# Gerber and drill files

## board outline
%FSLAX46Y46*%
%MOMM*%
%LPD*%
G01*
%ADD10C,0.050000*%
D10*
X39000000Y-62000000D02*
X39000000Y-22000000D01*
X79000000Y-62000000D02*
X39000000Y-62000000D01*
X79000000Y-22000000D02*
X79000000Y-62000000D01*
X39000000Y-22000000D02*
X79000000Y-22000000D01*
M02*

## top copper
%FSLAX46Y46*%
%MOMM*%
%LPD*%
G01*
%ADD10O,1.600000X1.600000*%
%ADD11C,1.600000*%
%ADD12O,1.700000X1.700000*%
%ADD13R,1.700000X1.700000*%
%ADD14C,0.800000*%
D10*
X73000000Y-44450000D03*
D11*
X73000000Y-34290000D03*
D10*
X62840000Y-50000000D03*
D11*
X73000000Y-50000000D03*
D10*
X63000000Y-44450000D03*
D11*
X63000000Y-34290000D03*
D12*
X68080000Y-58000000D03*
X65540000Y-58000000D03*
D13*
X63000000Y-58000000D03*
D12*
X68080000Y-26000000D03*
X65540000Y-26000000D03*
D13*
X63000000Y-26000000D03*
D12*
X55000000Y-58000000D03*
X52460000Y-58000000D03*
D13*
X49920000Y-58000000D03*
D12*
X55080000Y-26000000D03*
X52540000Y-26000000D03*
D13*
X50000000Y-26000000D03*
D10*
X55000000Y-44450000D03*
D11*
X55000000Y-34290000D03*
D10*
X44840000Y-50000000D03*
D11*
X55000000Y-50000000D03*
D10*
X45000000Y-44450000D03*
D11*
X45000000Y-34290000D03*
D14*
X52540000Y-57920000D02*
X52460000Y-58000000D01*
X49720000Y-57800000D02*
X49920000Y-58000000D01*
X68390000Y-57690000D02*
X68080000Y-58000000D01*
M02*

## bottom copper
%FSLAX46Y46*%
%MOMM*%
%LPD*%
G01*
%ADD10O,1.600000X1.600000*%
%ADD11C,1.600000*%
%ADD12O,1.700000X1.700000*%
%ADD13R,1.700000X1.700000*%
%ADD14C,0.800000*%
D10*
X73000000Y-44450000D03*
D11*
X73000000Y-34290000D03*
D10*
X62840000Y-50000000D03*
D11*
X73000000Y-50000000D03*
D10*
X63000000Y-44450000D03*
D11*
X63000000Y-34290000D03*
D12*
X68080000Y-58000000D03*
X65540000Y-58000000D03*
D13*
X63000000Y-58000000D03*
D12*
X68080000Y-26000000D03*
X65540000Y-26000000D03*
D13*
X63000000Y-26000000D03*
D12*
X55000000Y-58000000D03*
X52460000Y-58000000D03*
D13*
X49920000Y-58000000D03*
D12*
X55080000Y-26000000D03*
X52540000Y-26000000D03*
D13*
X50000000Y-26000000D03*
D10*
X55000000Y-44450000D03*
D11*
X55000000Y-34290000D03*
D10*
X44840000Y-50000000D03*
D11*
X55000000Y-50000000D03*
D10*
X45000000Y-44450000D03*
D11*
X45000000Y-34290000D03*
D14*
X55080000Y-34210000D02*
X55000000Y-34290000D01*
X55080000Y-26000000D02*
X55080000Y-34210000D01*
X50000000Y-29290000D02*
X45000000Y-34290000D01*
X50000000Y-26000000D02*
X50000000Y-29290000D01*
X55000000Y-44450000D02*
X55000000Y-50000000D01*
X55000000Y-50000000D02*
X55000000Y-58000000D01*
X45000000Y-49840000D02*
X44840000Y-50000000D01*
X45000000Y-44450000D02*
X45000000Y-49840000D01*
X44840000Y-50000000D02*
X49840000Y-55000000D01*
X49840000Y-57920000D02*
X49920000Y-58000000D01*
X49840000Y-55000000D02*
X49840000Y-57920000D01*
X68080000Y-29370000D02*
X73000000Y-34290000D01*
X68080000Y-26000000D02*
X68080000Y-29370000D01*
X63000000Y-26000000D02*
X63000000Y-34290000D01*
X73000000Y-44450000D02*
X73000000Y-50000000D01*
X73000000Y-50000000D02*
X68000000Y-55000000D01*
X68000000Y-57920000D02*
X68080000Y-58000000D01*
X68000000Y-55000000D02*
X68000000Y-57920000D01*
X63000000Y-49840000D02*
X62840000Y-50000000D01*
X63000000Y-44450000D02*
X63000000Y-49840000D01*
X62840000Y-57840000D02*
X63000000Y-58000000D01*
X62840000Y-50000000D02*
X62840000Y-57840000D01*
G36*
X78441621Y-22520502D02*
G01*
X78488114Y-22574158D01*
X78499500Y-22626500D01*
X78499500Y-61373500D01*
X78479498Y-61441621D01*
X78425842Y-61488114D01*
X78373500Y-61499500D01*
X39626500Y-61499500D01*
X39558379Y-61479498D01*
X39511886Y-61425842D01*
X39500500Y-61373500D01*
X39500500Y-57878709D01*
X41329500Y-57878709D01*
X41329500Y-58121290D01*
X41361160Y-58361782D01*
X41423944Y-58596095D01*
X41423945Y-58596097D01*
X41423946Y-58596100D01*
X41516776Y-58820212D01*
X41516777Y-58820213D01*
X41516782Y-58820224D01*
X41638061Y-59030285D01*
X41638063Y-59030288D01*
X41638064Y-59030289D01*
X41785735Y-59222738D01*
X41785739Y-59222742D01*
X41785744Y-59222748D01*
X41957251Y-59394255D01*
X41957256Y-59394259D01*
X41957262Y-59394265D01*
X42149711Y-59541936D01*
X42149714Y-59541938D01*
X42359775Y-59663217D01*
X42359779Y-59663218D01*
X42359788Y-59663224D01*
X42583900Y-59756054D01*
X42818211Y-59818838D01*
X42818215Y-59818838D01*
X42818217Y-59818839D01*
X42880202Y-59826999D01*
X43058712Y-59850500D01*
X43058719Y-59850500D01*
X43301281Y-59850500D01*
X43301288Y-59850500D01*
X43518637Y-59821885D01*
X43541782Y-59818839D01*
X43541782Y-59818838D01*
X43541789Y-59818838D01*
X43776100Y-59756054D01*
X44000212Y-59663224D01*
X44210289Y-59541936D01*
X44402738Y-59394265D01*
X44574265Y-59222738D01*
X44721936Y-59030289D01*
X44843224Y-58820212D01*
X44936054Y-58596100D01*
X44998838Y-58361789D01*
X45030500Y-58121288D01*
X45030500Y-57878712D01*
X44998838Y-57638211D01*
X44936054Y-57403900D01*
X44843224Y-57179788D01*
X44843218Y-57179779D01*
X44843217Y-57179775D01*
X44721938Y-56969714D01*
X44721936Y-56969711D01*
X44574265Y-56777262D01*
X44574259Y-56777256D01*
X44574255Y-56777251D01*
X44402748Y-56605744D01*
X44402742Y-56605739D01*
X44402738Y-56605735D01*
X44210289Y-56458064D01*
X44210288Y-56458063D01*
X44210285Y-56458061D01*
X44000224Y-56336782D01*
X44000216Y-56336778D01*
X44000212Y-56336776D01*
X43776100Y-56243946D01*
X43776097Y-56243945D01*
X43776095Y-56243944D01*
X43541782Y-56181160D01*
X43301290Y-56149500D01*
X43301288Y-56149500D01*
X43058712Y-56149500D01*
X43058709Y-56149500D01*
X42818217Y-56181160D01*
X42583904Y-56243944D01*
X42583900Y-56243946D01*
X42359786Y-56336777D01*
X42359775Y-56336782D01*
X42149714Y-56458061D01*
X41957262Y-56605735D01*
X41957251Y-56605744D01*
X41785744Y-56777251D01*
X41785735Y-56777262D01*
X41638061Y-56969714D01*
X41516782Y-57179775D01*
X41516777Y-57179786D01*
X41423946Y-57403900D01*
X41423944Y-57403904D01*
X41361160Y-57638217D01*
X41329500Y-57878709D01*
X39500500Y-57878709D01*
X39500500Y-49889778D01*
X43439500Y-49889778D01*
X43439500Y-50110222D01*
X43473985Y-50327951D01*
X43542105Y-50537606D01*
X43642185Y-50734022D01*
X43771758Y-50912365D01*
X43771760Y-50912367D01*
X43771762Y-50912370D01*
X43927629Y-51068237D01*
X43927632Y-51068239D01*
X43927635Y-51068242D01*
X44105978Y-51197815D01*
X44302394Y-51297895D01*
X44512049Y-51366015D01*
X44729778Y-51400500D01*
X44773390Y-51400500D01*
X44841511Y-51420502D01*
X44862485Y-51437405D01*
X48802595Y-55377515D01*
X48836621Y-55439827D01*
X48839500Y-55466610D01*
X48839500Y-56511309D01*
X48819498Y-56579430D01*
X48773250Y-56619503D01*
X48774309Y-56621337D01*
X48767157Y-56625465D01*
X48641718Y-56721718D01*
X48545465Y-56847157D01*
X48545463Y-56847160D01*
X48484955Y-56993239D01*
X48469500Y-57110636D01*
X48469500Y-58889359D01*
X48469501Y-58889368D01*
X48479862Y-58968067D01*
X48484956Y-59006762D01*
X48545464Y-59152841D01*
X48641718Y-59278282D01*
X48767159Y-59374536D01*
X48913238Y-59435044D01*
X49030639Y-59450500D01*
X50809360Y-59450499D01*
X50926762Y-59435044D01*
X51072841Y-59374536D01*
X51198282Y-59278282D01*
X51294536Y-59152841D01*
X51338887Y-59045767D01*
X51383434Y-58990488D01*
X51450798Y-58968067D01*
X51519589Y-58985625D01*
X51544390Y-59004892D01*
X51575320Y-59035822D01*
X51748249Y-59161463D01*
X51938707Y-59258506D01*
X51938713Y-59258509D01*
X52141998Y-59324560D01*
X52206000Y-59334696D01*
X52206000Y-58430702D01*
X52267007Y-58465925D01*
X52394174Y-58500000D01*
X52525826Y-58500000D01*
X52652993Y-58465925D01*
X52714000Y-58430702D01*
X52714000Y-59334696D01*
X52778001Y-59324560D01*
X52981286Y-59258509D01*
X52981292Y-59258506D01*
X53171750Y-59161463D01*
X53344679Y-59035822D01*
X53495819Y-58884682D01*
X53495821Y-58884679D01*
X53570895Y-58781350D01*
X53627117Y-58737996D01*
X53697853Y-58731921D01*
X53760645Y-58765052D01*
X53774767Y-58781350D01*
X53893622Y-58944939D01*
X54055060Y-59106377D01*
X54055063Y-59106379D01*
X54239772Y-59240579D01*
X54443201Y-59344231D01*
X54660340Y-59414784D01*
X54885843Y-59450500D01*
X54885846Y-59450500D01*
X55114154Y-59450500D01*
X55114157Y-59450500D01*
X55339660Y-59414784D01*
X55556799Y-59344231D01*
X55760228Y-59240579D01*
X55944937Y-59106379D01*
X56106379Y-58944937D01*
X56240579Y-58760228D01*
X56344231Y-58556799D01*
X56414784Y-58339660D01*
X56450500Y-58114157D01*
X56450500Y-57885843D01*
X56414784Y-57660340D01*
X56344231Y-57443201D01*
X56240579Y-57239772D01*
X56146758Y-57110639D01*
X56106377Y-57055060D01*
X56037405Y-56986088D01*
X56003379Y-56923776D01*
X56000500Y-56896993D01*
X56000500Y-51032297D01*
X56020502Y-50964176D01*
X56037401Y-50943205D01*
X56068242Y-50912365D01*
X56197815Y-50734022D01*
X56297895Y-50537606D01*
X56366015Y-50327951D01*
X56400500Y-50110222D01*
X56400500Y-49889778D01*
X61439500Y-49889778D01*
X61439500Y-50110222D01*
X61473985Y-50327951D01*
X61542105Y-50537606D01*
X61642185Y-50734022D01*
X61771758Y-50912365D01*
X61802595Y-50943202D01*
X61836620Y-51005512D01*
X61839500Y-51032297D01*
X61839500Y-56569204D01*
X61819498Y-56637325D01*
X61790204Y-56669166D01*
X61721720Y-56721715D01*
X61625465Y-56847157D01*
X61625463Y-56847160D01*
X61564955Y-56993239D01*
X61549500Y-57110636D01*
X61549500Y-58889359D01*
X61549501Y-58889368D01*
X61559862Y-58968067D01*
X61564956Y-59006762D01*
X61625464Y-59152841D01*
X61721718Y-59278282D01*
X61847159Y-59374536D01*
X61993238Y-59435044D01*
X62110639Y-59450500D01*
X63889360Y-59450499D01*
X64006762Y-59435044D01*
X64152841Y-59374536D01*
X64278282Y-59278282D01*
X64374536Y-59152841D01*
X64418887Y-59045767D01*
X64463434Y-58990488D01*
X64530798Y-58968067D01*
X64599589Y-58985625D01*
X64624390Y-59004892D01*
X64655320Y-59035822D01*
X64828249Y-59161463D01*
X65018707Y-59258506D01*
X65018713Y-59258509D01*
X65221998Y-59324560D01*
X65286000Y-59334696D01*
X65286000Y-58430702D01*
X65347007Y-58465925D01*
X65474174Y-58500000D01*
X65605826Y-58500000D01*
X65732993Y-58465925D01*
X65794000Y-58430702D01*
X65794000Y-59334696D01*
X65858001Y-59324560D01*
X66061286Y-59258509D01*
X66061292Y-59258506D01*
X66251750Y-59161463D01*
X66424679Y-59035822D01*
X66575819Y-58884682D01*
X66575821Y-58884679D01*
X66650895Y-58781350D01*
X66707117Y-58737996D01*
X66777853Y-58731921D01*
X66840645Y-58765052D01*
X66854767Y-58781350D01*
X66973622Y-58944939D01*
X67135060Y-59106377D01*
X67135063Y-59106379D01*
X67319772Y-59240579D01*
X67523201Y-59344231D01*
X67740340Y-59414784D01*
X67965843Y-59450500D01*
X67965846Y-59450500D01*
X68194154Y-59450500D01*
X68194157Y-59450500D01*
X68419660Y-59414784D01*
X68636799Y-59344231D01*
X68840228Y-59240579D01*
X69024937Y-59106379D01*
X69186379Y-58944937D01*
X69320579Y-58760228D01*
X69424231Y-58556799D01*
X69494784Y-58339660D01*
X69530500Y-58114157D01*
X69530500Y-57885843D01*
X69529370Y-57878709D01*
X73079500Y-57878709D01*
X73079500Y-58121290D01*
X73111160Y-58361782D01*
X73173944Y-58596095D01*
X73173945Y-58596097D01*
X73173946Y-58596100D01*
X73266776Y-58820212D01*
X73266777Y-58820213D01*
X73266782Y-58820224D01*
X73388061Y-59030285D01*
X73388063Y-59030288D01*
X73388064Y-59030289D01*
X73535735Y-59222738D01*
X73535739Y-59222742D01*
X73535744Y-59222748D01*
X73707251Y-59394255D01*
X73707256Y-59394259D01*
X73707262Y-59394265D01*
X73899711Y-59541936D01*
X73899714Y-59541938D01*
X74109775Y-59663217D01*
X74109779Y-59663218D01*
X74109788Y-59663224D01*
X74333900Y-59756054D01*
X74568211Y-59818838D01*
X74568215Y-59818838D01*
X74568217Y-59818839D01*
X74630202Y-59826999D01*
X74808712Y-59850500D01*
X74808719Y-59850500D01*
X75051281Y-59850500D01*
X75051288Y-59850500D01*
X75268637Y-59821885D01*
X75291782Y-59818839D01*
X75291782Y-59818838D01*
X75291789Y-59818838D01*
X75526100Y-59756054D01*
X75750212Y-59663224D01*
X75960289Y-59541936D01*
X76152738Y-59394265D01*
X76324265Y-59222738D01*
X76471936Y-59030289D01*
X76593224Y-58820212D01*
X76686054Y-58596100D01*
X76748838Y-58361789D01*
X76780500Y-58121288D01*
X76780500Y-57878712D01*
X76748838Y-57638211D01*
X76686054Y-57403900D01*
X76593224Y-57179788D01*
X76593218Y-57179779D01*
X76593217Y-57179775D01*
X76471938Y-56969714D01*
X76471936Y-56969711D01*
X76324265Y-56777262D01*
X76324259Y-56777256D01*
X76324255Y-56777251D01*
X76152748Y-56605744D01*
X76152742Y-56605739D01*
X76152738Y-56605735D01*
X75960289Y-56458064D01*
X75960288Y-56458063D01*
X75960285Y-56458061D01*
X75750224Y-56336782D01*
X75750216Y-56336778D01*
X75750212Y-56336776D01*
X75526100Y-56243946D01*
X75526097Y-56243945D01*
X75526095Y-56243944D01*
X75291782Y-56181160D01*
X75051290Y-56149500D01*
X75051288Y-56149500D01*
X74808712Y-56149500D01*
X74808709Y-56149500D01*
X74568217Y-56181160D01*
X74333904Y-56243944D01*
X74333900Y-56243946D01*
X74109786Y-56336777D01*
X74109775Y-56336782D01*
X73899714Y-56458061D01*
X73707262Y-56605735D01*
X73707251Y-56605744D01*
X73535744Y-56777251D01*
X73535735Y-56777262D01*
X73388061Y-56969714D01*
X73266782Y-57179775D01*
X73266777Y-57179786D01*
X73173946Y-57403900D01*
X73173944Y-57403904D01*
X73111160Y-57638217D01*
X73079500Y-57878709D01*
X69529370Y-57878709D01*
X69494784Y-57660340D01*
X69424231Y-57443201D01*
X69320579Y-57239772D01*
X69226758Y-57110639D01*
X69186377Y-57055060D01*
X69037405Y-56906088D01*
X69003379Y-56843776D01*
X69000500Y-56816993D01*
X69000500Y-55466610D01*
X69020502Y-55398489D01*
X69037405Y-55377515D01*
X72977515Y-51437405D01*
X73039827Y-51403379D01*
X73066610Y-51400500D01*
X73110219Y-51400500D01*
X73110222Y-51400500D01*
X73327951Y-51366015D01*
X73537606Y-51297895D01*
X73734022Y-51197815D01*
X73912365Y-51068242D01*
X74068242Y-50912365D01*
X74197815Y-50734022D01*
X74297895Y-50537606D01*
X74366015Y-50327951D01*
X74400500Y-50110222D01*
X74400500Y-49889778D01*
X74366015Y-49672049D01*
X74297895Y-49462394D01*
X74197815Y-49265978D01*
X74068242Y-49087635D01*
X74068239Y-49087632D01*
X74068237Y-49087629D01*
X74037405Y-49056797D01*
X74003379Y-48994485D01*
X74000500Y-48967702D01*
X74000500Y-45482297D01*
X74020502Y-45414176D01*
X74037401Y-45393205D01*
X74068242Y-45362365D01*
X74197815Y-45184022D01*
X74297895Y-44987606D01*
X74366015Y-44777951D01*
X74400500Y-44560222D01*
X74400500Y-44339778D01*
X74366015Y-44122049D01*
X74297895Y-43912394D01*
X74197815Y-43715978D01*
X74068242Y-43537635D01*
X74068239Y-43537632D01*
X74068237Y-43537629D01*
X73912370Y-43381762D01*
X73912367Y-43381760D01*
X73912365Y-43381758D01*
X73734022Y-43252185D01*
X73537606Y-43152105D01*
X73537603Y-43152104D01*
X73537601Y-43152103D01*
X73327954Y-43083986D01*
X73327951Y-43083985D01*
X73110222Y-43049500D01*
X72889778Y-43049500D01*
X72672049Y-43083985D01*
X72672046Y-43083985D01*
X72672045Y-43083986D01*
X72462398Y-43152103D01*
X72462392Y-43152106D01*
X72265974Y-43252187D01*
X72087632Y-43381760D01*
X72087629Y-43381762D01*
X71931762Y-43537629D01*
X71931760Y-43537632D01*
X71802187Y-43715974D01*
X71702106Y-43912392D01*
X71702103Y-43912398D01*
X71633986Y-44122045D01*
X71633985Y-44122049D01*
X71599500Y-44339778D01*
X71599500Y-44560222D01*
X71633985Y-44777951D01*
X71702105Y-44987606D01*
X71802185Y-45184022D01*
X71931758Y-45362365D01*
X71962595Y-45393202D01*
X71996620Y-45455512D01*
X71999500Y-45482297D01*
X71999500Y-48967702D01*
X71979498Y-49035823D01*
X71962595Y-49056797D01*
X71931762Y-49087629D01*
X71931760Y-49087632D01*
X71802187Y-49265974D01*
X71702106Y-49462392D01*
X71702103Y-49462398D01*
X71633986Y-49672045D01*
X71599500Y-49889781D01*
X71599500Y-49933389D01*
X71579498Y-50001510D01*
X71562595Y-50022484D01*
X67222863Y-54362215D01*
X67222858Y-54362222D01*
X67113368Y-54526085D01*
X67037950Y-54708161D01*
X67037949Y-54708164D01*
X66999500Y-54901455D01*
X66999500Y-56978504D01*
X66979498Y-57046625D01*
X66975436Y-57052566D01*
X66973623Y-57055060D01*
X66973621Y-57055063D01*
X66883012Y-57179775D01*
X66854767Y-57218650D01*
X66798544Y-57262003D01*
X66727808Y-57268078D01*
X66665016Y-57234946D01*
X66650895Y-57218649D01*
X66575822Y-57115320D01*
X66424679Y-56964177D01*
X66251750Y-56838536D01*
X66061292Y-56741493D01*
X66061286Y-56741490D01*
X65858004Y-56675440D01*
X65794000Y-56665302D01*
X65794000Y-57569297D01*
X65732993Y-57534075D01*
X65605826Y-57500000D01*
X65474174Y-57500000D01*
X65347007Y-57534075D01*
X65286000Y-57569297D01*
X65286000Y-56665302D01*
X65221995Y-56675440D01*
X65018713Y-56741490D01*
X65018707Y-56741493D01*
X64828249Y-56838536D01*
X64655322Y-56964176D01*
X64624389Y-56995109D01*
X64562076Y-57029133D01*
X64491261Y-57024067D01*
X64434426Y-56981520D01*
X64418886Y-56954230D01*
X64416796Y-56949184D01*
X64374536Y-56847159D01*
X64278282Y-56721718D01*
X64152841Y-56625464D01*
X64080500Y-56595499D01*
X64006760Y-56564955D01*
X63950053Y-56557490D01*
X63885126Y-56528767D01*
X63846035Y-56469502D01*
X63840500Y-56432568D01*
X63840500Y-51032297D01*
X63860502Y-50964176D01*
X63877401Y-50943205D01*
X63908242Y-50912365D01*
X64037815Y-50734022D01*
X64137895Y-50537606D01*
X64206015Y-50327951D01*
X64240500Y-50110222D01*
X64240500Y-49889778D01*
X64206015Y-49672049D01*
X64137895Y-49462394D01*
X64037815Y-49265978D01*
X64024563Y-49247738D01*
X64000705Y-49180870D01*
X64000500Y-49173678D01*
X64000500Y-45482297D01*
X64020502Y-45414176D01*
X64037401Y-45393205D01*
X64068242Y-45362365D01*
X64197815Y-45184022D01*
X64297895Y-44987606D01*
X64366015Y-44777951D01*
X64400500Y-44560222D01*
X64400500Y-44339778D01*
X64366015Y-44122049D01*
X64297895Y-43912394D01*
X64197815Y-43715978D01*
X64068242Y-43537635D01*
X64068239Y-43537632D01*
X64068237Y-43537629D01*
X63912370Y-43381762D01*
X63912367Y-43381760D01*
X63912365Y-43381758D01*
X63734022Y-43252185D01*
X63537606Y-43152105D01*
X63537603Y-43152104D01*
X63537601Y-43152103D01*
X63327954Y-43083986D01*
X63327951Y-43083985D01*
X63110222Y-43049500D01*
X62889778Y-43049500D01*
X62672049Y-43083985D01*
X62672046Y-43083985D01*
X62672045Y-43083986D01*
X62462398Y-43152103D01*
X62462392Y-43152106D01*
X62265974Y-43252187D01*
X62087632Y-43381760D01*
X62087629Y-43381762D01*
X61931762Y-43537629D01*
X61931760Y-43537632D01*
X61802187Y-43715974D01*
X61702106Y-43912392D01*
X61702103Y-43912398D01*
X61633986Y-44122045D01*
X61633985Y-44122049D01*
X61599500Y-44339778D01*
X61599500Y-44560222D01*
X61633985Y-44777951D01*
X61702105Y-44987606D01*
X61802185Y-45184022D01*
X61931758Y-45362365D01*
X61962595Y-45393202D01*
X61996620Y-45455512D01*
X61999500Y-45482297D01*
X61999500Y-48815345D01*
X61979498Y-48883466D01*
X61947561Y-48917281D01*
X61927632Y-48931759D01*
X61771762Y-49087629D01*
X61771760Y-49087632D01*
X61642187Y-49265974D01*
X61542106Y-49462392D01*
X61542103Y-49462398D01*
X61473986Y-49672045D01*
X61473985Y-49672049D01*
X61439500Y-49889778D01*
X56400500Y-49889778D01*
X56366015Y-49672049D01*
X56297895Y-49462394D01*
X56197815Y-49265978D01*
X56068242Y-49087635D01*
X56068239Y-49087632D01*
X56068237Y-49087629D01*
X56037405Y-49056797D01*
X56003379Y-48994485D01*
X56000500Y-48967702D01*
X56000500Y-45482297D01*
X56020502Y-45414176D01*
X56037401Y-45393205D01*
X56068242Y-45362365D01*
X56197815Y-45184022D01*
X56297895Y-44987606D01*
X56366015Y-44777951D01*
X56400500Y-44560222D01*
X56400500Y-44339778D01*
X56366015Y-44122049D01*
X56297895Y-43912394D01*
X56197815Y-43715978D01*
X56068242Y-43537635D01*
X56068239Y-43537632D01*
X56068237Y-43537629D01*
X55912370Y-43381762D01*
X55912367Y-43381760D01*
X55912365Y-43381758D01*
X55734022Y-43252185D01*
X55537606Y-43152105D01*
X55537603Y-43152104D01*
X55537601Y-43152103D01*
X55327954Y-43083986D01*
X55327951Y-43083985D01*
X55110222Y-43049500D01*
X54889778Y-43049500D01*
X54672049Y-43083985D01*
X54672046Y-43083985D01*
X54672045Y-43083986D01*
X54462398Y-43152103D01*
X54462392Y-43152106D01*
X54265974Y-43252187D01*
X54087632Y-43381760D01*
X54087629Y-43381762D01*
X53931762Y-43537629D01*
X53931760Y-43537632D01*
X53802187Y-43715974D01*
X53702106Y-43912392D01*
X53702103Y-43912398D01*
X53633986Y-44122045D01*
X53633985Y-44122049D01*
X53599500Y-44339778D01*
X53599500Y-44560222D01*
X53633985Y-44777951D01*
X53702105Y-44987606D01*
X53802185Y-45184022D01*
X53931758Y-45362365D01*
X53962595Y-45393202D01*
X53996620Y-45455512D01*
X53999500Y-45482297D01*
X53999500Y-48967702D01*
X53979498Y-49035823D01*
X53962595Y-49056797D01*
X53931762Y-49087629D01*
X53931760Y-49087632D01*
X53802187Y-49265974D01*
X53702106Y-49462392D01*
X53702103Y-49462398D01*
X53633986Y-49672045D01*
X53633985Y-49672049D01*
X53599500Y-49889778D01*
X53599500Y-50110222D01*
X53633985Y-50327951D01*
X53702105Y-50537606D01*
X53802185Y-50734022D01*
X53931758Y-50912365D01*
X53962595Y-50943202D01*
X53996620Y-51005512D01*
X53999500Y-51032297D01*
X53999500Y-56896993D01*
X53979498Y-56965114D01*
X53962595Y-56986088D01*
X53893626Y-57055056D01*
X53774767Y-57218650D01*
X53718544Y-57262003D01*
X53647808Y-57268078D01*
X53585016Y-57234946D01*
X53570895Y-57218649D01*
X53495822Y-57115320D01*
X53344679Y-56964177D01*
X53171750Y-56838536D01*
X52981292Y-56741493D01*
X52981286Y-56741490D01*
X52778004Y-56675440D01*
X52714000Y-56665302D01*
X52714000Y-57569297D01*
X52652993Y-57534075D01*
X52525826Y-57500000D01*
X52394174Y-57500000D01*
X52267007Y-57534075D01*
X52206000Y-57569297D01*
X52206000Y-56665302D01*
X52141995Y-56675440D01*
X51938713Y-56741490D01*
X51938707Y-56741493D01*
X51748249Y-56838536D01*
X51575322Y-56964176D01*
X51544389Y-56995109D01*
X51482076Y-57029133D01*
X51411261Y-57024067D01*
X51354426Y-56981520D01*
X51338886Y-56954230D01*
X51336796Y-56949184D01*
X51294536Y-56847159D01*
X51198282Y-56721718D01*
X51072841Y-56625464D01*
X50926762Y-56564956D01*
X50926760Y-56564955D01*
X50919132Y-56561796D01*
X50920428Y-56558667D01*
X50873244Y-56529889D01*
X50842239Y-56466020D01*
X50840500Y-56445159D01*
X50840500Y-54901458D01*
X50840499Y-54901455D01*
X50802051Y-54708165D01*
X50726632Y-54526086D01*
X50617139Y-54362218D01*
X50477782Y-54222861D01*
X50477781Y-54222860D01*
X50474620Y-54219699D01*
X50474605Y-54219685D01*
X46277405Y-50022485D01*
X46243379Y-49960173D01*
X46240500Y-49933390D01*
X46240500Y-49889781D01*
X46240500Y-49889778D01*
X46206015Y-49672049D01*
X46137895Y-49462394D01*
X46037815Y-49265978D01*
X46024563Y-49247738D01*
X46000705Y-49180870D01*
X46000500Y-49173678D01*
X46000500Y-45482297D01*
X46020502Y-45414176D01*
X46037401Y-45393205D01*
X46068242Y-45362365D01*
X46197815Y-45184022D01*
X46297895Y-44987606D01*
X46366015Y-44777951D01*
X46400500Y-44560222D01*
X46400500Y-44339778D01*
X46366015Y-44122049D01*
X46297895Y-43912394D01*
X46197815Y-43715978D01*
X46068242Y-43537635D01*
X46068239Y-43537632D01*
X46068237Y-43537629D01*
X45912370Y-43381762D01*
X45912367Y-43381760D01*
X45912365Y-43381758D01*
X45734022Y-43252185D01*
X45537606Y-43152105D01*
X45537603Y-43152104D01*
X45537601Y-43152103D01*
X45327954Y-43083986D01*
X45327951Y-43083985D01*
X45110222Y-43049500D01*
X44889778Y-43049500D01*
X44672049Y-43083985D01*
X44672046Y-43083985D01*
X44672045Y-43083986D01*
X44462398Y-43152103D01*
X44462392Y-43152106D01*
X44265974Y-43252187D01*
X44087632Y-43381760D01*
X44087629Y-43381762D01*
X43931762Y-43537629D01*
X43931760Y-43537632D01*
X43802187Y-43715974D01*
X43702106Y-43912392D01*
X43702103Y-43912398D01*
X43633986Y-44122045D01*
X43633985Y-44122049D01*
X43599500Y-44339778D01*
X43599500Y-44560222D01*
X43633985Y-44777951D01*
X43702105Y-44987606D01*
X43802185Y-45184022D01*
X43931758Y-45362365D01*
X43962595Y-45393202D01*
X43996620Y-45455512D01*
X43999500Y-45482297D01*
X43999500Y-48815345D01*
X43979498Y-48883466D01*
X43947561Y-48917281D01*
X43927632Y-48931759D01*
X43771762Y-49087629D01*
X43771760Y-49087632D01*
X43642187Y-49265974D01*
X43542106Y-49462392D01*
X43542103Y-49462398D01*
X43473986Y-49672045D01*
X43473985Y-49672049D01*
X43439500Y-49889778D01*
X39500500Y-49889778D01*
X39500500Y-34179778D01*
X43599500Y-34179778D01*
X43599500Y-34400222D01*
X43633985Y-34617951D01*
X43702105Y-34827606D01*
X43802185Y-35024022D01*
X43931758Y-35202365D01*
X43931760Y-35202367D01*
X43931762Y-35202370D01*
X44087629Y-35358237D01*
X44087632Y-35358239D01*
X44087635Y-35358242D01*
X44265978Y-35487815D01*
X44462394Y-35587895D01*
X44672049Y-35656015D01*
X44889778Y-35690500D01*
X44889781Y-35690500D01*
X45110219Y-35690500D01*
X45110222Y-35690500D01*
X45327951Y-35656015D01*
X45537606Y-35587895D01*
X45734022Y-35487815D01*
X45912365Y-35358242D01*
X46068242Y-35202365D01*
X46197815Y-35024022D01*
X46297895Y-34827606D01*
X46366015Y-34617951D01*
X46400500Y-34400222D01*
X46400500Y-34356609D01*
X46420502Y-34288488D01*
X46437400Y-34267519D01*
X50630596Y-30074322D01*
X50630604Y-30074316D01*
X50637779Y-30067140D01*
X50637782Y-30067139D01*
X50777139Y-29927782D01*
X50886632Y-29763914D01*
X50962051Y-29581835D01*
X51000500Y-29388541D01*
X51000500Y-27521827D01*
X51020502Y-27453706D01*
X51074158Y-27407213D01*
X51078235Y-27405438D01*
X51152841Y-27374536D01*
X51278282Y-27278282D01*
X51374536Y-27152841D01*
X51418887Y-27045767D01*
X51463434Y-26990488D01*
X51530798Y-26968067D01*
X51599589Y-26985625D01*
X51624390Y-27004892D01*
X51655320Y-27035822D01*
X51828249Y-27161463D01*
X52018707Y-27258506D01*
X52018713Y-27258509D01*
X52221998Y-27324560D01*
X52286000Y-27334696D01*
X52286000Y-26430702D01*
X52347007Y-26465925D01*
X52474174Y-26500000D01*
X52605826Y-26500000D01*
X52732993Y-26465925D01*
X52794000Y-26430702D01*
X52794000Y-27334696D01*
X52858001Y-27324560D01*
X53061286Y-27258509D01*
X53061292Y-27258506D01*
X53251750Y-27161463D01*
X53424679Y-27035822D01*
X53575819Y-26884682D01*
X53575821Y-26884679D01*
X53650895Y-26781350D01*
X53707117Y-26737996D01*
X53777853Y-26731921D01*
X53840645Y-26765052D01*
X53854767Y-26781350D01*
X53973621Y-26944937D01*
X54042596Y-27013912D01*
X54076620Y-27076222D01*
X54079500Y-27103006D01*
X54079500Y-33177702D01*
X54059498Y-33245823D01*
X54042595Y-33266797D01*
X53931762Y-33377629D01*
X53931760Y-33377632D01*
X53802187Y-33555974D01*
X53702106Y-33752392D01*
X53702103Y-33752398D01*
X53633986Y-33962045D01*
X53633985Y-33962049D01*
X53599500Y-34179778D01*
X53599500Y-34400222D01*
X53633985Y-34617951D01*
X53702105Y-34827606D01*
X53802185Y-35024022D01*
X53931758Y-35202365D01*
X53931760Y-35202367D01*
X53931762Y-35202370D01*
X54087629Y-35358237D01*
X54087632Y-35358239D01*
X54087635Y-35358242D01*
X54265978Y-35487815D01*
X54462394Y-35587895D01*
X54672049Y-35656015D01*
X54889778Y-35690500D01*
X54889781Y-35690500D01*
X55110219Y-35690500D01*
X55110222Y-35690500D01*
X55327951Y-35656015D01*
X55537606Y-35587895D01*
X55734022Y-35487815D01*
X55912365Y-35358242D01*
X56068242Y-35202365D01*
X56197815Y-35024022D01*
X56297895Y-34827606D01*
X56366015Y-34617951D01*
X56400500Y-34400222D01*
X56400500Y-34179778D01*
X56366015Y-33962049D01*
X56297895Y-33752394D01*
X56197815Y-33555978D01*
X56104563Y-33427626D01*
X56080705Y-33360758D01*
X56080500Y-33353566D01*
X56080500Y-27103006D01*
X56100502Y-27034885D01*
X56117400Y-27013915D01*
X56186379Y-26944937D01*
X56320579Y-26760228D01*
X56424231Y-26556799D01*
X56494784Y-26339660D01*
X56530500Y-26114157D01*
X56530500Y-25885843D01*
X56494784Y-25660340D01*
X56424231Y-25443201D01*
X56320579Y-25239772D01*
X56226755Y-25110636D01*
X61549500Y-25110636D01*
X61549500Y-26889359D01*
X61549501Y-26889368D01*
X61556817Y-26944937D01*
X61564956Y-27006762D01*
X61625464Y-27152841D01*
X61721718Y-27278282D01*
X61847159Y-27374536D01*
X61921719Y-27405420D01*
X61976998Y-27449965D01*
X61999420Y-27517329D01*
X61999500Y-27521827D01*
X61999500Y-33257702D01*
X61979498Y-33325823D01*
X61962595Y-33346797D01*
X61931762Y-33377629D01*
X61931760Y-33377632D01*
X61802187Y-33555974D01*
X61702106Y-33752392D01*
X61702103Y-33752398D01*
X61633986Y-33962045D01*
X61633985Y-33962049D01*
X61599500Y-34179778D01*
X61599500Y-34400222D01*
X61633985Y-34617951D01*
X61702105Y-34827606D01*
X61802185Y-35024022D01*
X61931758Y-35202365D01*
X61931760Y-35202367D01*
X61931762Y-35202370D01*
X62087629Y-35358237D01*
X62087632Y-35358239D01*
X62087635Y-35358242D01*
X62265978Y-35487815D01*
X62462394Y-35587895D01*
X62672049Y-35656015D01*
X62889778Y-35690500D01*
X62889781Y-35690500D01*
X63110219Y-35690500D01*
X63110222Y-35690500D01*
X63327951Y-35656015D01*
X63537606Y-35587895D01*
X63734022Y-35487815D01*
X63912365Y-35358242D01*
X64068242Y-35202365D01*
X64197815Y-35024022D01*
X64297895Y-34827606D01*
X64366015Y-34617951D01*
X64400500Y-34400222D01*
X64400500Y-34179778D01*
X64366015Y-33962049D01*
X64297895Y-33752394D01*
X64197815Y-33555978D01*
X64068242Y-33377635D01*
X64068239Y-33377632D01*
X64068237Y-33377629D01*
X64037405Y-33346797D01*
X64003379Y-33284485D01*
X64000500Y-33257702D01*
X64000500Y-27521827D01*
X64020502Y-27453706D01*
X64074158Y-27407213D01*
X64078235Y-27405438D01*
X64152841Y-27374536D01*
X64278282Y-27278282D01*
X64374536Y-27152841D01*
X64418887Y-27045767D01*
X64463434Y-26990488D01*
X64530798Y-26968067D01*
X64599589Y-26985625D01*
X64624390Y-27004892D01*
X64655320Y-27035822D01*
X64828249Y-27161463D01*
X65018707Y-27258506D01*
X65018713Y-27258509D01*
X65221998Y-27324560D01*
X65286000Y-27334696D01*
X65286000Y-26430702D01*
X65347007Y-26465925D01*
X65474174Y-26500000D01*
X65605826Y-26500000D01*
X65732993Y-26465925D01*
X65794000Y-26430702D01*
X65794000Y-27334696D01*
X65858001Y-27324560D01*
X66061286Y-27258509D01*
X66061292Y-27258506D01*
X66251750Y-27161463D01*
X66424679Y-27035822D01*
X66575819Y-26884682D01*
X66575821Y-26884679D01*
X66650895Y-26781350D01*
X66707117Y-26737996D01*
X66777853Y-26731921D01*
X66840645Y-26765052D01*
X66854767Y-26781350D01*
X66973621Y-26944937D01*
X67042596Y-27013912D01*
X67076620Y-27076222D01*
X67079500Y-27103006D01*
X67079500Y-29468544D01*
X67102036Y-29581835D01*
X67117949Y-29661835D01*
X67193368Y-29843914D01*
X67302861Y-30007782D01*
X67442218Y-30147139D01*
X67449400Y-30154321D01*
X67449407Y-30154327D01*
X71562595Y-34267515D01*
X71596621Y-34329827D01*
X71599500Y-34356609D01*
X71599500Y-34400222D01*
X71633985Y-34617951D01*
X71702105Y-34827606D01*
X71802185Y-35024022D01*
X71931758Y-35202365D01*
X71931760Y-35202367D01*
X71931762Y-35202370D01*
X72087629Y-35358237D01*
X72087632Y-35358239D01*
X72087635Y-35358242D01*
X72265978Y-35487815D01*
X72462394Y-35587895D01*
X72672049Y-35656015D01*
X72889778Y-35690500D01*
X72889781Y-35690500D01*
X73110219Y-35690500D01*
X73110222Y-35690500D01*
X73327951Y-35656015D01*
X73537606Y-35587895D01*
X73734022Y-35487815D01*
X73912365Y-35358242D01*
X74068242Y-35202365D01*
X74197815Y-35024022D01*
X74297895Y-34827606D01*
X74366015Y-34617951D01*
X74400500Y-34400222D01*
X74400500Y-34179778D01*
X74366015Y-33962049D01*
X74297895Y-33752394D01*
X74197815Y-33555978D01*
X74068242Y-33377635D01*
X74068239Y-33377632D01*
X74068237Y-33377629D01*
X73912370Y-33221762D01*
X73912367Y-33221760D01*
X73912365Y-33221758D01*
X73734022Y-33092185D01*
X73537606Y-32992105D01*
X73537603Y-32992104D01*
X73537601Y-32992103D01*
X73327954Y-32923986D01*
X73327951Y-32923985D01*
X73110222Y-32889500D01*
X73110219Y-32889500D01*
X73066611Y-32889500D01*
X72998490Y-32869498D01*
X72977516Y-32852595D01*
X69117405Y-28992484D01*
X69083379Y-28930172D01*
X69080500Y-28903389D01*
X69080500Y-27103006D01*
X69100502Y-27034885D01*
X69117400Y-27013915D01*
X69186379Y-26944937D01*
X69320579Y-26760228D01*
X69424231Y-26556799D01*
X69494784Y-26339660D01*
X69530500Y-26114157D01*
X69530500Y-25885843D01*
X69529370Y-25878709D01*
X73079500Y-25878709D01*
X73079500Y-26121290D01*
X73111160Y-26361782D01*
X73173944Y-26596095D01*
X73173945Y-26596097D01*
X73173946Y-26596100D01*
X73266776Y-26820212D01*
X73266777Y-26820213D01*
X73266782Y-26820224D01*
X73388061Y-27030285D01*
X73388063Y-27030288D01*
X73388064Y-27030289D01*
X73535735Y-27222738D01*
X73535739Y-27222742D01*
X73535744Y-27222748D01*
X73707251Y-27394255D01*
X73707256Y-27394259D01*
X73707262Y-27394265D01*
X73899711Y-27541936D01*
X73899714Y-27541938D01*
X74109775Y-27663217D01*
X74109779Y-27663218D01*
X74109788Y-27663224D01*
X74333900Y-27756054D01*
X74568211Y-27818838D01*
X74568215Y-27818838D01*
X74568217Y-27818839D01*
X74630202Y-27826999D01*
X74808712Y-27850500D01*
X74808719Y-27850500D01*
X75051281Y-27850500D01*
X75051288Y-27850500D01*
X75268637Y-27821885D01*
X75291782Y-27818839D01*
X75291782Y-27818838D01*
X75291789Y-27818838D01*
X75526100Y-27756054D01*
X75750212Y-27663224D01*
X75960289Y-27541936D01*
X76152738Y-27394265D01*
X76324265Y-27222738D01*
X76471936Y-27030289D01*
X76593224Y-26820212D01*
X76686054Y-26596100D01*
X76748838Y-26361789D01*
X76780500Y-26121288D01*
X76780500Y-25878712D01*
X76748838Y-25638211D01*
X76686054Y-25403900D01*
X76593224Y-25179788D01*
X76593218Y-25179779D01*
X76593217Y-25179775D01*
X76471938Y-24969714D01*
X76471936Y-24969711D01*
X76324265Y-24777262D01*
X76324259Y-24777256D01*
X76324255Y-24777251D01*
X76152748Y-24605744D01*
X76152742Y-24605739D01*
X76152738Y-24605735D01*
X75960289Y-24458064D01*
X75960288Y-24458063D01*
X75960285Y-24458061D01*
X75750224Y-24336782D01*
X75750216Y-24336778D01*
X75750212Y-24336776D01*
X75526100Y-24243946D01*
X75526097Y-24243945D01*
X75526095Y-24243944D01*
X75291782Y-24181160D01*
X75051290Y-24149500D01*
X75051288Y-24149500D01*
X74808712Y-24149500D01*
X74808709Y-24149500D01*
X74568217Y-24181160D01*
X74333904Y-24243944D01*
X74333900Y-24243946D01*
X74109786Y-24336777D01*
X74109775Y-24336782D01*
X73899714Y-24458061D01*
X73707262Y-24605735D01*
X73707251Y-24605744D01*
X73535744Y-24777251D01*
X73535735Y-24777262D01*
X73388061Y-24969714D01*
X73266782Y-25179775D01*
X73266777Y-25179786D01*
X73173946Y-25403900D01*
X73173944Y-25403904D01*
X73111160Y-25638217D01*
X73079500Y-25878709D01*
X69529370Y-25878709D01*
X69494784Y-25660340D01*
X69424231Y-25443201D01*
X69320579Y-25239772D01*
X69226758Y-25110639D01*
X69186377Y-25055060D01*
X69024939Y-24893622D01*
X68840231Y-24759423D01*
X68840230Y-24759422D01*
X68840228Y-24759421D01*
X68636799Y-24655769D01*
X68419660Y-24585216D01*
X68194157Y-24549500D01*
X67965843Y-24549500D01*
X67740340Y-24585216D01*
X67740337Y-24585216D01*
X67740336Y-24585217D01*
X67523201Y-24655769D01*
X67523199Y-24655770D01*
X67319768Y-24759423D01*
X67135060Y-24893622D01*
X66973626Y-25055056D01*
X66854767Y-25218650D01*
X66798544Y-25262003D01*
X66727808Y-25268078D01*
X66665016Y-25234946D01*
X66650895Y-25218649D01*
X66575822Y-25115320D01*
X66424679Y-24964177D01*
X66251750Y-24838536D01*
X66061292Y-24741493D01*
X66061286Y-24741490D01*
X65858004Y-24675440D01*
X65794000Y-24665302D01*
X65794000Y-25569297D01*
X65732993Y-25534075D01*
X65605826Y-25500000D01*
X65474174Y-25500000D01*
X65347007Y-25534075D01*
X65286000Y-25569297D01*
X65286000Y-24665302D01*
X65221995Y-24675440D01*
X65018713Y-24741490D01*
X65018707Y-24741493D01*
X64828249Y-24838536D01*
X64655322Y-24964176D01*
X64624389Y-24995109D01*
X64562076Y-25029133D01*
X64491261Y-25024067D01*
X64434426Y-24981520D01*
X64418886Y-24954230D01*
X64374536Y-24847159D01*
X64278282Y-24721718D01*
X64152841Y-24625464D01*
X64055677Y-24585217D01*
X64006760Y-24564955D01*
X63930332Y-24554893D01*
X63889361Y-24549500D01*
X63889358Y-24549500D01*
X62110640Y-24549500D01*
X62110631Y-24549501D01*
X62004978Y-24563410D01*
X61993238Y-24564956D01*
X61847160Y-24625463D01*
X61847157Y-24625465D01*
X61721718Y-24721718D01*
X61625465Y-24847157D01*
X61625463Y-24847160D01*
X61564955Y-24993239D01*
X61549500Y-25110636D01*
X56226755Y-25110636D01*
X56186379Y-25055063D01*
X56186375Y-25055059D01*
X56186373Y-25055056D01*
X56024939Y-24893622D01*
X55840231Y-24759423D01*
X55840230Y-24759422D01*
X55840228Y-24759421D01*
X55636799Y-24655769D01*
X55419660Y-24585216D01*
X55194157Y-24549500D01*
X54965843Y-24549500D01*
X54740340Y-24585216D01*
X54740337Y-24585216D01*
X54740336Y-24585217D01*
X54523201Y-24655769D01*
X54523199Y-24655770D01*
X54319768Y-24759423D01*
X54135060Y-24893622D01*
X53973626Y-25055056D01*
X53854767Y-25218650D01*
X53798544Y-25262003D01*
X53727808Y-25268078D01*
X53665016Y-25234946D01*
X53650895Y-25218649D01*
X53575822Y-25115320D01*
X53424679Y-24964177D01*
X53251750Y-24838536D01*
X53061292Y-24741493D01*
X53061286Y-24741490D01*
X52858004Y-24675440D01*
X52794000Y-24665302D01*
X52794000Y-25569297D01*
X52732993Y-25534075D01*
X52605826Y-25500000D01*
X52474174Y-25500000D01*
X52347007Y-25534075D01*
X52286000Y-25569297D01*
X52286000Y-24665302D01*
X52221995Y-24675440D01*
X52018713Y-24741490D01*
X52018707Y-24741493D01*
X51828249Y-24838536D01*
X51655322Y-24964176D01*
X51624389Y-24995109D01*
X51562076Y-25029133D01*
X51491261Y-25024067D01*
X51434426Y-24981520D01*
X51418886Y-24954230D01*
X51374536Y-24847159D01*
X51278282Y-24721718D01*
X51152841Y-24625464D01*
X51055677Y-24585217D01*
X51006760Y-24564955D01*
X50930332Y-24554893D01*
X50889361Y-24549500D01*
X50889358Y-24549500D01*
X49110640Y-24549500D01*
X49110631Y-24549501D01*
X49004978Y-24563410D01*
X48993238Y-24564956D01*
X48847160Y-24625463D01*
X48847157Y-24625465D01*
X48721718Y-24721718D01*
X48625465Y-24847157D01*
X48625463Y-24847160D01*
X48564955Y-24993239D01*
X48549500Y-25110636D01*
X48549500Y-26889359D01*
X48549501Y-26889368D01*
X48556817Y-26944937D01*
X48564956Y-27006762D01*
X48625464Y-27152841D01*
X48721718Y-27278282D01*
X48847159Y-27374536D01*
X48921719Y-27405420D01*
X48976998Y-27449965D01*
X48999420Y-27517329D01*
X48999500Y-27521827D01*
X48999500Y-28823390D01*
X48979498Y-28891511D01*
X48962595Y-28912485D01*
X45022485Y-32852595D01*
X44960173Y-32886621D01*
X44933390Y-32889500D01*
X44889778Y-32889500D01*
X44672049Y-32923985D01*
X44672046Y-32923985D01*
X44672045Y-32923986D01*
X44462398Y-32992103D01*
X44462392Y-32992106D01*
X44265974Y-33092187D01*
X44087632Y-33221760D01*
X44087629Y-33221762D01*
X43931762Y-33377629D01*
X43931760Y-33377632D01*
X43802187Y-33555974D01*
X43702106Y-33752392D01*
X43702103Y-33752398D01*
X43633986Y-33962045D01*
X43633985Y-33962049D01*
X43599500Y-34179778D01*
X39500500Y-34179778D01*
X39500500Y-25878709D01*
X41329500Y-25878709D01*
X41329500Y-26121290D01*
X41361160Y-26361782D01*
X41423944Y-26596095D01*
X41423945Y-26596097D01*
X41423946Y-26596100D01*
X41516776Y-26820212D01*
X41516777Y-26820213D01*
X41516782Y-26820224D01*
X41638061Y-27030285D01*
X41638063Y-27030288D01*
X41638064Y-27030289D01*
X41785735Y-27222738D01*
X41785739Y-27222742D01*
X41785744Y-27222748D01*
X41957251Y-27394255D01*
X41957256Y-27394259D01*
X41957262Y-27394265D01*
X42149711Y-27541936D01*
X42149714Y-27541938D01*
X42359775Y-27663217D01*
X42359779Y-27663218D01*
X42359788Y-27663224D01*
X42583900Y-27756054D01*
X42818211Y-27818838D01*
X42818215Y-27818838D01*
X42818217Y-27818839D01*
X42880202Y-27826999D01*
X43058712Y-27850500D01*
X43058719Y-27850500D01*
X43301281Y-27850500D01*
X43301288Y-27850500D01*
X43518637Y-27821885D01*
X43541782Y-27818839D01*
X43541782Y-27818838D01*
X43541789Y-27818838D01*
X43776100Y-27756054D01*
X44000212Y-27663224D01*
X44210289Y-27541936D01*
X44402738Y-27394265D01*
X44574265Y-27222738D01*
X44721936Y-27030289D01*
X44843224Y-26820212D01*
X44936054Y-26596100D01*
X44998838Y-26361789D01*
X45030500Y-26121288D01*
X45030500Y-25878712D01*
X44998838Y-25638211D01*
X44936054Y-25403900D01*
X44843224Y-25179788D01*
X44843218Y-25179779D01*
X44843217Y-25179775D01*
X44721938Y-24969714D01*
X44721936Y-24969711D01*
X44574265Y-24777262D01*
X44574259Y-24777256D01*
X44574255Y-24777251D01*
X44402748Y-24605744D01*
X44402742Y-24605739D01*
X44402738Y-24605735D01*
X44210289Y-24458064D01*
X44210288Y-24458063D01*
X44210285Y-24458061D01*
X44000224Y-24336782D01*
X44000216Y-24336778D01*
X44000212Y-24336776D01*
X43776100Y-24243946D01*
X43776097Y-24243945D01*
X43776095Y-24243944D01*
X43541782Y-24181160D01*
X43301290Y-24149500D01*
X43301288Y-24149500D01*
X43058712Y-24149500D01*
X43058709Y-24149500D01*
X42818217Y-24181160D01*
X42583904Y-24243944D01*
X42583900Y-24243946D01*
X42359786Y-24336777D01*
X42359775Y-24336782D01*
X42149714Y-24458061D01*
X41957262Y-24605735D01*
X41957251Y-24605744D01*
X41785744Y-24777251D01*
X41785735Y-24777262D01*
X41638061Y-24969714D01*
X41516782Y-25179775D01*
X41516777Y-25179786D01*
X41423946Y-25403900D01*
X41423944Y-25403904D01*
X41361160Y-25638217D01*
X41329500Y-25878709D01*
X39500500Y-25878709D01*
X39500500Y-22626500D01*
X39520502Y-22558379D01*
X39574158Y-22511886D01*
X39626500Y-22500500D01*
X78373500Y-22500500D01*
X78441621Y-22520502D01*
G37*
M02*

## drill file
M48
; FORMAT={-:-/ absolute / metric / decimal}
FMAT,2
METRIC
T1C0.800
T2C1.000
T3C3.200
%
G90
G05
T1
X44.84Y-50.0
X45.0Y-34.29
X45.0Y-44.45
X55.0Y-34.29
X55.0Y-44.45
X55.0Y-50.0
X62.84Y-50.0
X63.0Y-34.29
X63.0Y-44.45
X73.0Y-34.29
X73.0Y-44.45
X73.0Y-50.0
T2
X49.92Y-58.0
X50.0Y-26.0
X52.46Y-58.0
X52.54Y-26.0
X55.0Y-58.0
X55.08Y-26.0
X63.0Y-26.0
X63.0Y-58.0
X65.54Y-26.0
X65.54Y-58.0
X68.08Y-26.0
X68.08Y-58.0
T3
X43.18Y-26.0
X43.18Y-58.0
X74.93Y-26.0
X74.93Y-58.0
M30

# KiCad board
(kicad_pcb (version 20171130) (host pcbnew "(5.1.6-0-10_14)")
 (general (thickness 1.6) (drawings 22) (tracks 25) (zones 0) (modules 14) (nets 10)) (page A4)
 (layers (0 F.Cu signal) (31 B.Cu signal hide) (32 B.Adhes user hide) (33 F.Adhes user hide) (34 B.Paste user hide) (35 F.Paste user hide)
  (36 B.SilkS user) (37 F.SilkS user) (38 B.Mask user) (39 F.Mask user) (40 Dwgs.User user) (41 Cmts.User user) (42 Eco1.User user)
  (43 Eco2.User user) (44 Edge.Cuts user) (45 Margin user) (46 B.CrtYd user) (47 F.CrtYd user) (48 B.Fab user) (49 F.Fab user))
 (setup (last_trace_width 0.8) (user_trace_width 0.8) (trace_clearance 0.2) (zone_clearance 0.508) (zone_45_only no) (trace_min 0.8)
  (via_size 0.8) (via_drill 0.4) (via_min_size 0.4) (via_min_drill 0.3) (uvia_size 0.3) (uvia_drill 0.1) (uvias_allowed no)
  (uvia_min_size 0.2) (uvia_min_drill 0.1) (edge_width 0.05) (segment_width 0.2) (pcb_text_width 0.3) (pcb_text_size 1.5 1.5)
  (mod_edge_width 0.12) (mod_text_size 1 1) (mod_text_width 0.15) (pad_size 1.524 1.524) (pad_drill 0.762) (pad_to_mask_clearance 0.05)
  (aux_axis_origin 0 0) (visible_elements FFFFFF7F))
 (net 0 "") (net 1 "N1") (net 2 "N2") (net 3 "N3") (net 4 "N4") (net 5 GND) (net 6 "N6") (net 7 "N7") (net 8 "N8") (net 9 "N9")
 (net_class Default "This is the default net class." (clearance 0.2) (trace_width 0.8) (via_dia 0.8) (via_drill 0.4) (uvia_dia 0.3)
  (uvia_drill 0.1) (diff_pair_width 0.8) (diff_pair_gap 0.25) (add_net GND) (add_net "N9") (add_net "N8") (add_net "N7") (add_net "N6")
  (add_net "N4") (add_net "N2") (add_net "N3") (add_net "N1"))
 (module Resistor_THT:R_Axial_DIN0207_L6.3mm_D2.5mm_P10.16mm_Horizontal (layer F.Cu) (at 73 34.29 270)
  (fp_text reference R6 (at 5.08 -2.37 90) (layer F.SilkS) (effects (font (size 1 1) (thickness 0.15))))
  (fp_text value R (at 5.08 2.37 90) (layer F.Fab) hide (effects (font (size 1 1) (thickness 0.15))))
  (pad 2 thru_hole oval (at 10.16 0 270) (size 1.6 1.6) (drill 0.8) (layers *.Cu *.Mask) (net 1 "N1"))
  (pad 1 thru_hole circle (at 0 0 270) (size 1.6 1.6) (drill 0.8) (layers *.Cu *.Mask) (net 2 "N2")))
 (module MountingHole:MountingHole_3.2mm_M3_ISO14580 (layer F.Cu) (at 43.18 26)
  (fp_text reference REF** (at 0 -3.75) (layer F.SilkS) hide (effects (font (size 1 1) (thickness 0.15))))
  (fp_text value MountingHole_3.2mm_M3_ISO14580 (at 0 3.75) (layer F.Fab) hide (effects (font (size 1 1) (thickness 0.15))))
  (pad 1 np_thru_hole circle (at 0 0) (size 3.2 3.2) (drill 3.2) (layers *.Cu *.Mask)))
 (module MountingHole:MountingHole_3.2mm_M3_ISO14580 (layer F.Cu) (at 74.93 58)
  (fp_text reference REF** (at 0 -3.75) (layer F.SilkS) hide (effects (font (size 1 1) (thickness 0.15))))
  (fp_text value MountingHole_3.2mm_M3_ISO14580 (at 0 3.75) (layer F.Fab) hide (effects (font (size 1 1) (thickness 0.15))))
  (pad 1 np_thru_hole circle (at 0 0) (size 3.2 3.2) (drill 3.2) (layers *.Cu *.Mask)))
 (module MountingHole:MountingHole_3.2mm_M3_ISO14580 (layer F.Cu) (at 43.18 58)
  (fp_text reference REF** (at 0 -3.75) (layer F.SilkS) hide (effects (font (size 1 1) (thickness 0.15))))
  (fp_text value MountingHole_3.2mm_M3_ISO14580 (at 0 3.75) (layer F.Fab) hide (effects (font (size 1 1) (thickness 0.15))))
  (pad 1 np_thru_hole circle (at 0 0) (size 3.2 3.2) (drill 3.2) (layers *.Cu *.Mask)))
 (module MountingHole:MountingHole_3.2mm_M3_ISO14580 (layer F.Cu) (at 74.93 26)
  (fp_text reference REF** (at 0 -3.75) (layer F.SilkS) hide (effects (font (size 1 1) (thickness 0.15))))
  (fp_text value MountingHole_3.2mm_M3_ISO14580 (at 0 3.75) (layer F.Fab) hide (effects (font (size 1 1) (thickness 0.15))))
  (pad 1 np_thru_hole circle (at 0 0) (size 3.2 3.2) (drill 3.2) (layers *.Cu *.Mask)))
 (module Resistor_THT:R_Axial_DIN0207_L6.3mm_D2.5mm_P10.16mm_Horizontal (layer F.Cu) (at 73 50 180)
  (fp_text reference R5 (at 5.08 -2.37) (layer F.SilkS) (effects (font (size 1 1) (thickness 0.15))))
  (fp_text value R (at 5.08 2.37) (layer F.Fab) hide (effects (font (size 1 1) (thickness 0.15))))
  (pad 2 thru_hole oval (at 10.16 0 180) (size 1.6 1.6) (drill 0.8) (layers *.Cu *.Mask) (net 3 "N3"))
  (pad 1 thru_hole circle (at 0 0 180) (size 1.6 1.6) (drill 0.8) (layers *.Cu *.Mask) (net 1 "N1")))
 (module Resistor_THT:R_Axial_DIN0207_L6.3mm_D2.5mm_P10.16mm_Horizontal (layer F.Cu) (at 63 34.29 270)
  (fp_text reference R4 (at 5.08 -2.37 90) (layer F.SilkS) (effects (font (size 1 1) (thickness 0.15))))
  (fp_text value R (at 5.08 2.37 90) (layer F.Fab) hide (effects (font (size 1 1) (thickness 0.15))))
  (pad 2 thru_hole oval (at 10.16 0 270) (size 1.6 1.6) (drill 0.8) (layers *.Cu *.Mask) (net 3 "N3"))
  (pad 1 thru_hole circle (at 0 0 270) (size 1.6 1.6) (drill 0.8) (layers *.Cu *.Mask) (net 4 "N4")))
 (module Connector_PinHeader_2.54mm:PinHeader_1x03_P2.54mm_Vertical (layer F.Cu) (at 63 58 90)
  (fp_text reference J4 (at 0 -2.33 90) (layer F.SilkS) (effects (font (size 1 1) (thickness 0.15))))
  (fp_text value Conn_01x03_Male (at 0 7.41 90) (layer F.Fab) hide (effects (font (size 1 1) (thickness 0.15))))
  (pad 3 thru_hole oval (at 0 5.08 90) (size 1.7 1.7) (drill 1) (layers *.Cu *.Mask) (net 1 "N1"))
  (pad 2 thru_hole oval (at 0 2.54 90) (size 1.7 1.7) (drill 1) (layers *.Cu *.Mask) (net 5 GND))
  (pad 1 thru_hole rect (at 0 0 90) (size 1.7 1.7) (drill 1) (layers *.Cu *.Mask) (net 3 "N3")))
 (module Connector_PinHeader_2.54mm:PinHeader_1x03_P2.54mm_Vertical (layer F.Cu) (at 63 26 90)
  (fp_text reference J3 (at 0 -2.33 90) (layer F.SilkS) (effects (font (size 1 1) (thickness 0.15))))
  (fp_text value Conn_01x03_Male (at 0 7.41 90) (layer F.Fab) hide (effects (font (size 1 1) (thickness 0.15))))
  (pad 3 thru_hole oval (at 0 5.08 90) (size 1.7 1.7) (drill 1) (layers *.Cu *.Mask) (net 2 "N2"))
  (pad 2 thru_hole oval (at 0 2.54 90) (size 1.7 1.7) (drill 1) (layers *.Cu *.Mask) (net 5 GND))
  (pad 1 thru_hole rect (at 0 0 90) (size 1.7 1.7) (drill 1) (layers *.Cu *.Mask) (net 4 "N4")))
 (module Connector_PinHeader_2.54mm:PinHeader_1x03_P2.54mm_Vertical (layer F.Cu) (at 49.92 58 90)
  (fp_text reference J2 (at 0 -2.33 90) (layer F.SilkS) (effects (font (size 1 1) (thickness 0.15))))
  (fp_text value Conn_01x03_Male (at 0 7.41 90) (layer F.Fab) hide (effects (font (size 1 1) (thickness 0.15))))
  (pad 3 thru_hole oval (at 0 5.08 90) (size 1.7 1.7) (drill 1) (layers *.Cu *.Mask) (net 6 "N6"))
  (pad 2 thru_hole oval (at 0 2.54 90) (size 1.7 1.7) (drill 1) (layers *.Cu *.Mask) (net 5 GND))
  (pad 1 thru_hole rect (at 0 0 90) (size 1.7 1.7) (drill 1) (layers *.Cu *.Mask) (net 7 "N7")))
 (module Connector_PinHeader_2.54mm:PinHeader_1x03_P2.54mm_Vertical (layer F.Cu) (at 50 26 90)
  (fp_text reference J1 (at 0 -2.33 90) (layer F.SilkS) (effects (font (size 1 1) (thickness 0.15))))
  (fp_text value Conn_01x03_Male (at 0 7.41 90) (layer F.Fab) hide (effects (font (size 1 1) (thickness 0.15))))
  (pad 3 thru_hole oval (at 0 5.08 90) (size 1.7 1.7) (drill 1) (layers *.Cu *.Mask) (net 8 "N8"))
  (pad 2 thru_hole oval (at 0 2.54 90) (size 1.7 1.7) (drill 1) (layers *.Cu *.Mask) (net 5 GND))
  (pad 1 thru_hole rect (at 0 0 90) (size 1.7 1.7) (drill 1) (layers *.Cu *.Mask) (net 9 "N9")))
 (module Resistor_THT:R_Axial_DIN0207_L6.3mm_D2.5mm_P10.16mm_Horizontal (layer F.Cu) (at 55 34.29 270)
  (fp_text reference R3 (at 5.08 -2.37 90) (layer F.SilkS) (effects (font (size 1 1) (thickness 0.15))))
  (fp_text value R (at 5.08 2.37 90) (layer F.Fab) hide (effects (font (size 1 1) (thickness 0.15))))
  (pad 2 thru_hole oval (at 10.16 0 270) (size 1.6 1.6) (drill 0.8) (layers *.Cu *.Mask) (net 6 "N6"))
  (pad 1 thru_hole circle (at 0 0 270) (size 1.6 1.6) (drill 0.8) (layers *.Cu *.Mask) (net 8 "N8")))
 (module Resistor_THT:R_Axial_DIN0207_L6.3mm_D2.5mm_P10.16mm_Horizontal (layer F.Cu) (at 55 50 180)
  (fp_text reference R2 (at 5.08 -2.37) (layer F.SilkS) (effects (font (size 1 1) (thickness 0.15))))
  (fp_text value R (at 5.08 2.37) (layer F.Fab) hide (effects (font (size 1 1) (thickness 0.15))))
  (pad 2 thru_hole oval (at 10.16 0 180) (size 1.6 1.6) (drill 0.8) (layers *.Cu *.Mask) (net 7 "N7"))
  (pad 1 thru_hole circle (at 0 0 180) (size 1.6 1.6) (drill 0.8) (layers *.Cu *.Mask) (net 6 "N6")))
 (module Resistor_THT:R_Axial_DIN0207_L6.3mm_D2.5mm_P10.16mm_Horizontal (layer F.Cu) (at 45 34.29 270)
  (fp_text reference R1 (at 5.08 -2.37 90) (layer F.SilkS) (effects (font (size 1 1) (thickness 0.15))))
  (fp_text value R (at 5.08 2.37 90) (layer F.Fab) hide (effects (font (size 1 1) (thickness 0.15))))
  (pad 2 thru_hole oval (at 10.16 0 270) (size 1.6 1.6) (drill 0.8) (layers *.Cu *.Mask) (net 7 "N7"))
  (pad 1 thru_hole circle (at 0 0 270) (size 1.6 1.6) (drill 0.8) (layers *.Cu *.Mask) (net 9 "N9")))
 (gr_line (start 39 62) (end 39 22) (layer Edge.Cuts) (width 0.05))
 (gr_line (start 79 62) (end 39 62) (layer Edge.Cuts) (width 0.05))
 (gr_line (start 79 22) (end 79 62) (layer Edge.Cuts) (width 0.05))
 (gr_line (start 39 22) (end 79 22) (layer Edge.Cuts) (width 0.05))
 (segment (start 55.08 34.21) (end 55 34.29) (width 0.8) (layer B.Cu) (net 8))
 (segment (start 55.08 26) (end 55.08 34.21) (width 0.8) (layer B.Cu) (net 8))
 (segment (start 52.54 57.92) (end 52.46 58) (width 0.8) (layer F.Cu) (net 5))
 (segment (start 50 29.29) (end 45 34.29) (width 0.8) (layer B.Cu) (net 9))
 (segment (start 50 26) (end 50 29.29) (width 0.8) (layer B.Cu) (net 9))
 (segment (start 55 44.45) (end 55 50) (width 0.8) (layer B.Cu) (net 6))
 (segment (start 55 50) (end 55 58) (width 0.8) (layer B.Cu) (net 6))
 (segment (start 49.72 57.8) (end 49.92 58) (width 0.8) (layer F.Cu) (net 7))
 (segment (start 45 49.84) (end 44.84 50) (width 0.8) (layer B.Cu) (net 7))
 (segment (start 45 44.45) (end 45 49.84) (width 0.8) (layer B.Cu) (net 7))
 (segment (start 44.84 50) (end 49.84 55) (width 0.8) (layer B.Cu) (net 7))
 (segment (start 49.84 57.92) (end 49.92 58) (width 0.8) (layer B.Cu) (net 7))
 (segment (start 49.84 55) (end 49.84 57.92) (width 0.8) (layer B.Cu) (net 7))
 (segment (start 68.08 29.37) (end 73 34.29) (width 0.8) (layer B.Cu) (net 2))
 (segment (start 68.08 26) (end 68.08 29.37) (width 0.8) (layer B.Cu) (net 2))
 (segment (start 63 26) (end 63 34.29) (width 0.8) (layer B.Cu) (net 4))
 (segment (start 68.39 57.69) (end 68.08 58) (width 0.8) (layer F.Cu) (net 1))
 (segment (start 73 44.45) (end 73 50) (width 0.8) (layer B.Cu) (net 1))
 (segment (start 73 50) (end 68 55) (width 0.8) (layer B.Cu) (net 1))
 (segment (start 68 57.92) (end 68.08 58) (width 0.8) (layer B.Cu) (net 1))
 (segment (start 68 55) (end 68 57.92) (width 0.8) (layer B.Cu) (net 1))
 (segment (start 63 49.84) (end 62.84 50) (width 0.8) (layer B.Cu) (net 3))
 (segment (start 63 44.45) (end 63 49.84) (width 0.8) (layer B.Cu) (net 3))
 (segment (start 62.84 57.84) (end 63 58) (width 0.8) (layer B.Cu) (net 3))
 (segment (start 62.84 50) (end 62.84 57.84) (width 0.8) (layer B.Cu) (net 3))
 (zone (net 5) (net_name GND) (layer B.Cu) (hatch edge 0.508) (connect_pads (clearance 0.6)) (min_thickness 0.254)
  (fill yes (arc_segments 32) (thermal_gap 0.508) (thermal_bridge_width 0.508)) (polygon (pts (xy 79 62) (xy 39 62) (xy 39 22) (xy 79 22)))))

